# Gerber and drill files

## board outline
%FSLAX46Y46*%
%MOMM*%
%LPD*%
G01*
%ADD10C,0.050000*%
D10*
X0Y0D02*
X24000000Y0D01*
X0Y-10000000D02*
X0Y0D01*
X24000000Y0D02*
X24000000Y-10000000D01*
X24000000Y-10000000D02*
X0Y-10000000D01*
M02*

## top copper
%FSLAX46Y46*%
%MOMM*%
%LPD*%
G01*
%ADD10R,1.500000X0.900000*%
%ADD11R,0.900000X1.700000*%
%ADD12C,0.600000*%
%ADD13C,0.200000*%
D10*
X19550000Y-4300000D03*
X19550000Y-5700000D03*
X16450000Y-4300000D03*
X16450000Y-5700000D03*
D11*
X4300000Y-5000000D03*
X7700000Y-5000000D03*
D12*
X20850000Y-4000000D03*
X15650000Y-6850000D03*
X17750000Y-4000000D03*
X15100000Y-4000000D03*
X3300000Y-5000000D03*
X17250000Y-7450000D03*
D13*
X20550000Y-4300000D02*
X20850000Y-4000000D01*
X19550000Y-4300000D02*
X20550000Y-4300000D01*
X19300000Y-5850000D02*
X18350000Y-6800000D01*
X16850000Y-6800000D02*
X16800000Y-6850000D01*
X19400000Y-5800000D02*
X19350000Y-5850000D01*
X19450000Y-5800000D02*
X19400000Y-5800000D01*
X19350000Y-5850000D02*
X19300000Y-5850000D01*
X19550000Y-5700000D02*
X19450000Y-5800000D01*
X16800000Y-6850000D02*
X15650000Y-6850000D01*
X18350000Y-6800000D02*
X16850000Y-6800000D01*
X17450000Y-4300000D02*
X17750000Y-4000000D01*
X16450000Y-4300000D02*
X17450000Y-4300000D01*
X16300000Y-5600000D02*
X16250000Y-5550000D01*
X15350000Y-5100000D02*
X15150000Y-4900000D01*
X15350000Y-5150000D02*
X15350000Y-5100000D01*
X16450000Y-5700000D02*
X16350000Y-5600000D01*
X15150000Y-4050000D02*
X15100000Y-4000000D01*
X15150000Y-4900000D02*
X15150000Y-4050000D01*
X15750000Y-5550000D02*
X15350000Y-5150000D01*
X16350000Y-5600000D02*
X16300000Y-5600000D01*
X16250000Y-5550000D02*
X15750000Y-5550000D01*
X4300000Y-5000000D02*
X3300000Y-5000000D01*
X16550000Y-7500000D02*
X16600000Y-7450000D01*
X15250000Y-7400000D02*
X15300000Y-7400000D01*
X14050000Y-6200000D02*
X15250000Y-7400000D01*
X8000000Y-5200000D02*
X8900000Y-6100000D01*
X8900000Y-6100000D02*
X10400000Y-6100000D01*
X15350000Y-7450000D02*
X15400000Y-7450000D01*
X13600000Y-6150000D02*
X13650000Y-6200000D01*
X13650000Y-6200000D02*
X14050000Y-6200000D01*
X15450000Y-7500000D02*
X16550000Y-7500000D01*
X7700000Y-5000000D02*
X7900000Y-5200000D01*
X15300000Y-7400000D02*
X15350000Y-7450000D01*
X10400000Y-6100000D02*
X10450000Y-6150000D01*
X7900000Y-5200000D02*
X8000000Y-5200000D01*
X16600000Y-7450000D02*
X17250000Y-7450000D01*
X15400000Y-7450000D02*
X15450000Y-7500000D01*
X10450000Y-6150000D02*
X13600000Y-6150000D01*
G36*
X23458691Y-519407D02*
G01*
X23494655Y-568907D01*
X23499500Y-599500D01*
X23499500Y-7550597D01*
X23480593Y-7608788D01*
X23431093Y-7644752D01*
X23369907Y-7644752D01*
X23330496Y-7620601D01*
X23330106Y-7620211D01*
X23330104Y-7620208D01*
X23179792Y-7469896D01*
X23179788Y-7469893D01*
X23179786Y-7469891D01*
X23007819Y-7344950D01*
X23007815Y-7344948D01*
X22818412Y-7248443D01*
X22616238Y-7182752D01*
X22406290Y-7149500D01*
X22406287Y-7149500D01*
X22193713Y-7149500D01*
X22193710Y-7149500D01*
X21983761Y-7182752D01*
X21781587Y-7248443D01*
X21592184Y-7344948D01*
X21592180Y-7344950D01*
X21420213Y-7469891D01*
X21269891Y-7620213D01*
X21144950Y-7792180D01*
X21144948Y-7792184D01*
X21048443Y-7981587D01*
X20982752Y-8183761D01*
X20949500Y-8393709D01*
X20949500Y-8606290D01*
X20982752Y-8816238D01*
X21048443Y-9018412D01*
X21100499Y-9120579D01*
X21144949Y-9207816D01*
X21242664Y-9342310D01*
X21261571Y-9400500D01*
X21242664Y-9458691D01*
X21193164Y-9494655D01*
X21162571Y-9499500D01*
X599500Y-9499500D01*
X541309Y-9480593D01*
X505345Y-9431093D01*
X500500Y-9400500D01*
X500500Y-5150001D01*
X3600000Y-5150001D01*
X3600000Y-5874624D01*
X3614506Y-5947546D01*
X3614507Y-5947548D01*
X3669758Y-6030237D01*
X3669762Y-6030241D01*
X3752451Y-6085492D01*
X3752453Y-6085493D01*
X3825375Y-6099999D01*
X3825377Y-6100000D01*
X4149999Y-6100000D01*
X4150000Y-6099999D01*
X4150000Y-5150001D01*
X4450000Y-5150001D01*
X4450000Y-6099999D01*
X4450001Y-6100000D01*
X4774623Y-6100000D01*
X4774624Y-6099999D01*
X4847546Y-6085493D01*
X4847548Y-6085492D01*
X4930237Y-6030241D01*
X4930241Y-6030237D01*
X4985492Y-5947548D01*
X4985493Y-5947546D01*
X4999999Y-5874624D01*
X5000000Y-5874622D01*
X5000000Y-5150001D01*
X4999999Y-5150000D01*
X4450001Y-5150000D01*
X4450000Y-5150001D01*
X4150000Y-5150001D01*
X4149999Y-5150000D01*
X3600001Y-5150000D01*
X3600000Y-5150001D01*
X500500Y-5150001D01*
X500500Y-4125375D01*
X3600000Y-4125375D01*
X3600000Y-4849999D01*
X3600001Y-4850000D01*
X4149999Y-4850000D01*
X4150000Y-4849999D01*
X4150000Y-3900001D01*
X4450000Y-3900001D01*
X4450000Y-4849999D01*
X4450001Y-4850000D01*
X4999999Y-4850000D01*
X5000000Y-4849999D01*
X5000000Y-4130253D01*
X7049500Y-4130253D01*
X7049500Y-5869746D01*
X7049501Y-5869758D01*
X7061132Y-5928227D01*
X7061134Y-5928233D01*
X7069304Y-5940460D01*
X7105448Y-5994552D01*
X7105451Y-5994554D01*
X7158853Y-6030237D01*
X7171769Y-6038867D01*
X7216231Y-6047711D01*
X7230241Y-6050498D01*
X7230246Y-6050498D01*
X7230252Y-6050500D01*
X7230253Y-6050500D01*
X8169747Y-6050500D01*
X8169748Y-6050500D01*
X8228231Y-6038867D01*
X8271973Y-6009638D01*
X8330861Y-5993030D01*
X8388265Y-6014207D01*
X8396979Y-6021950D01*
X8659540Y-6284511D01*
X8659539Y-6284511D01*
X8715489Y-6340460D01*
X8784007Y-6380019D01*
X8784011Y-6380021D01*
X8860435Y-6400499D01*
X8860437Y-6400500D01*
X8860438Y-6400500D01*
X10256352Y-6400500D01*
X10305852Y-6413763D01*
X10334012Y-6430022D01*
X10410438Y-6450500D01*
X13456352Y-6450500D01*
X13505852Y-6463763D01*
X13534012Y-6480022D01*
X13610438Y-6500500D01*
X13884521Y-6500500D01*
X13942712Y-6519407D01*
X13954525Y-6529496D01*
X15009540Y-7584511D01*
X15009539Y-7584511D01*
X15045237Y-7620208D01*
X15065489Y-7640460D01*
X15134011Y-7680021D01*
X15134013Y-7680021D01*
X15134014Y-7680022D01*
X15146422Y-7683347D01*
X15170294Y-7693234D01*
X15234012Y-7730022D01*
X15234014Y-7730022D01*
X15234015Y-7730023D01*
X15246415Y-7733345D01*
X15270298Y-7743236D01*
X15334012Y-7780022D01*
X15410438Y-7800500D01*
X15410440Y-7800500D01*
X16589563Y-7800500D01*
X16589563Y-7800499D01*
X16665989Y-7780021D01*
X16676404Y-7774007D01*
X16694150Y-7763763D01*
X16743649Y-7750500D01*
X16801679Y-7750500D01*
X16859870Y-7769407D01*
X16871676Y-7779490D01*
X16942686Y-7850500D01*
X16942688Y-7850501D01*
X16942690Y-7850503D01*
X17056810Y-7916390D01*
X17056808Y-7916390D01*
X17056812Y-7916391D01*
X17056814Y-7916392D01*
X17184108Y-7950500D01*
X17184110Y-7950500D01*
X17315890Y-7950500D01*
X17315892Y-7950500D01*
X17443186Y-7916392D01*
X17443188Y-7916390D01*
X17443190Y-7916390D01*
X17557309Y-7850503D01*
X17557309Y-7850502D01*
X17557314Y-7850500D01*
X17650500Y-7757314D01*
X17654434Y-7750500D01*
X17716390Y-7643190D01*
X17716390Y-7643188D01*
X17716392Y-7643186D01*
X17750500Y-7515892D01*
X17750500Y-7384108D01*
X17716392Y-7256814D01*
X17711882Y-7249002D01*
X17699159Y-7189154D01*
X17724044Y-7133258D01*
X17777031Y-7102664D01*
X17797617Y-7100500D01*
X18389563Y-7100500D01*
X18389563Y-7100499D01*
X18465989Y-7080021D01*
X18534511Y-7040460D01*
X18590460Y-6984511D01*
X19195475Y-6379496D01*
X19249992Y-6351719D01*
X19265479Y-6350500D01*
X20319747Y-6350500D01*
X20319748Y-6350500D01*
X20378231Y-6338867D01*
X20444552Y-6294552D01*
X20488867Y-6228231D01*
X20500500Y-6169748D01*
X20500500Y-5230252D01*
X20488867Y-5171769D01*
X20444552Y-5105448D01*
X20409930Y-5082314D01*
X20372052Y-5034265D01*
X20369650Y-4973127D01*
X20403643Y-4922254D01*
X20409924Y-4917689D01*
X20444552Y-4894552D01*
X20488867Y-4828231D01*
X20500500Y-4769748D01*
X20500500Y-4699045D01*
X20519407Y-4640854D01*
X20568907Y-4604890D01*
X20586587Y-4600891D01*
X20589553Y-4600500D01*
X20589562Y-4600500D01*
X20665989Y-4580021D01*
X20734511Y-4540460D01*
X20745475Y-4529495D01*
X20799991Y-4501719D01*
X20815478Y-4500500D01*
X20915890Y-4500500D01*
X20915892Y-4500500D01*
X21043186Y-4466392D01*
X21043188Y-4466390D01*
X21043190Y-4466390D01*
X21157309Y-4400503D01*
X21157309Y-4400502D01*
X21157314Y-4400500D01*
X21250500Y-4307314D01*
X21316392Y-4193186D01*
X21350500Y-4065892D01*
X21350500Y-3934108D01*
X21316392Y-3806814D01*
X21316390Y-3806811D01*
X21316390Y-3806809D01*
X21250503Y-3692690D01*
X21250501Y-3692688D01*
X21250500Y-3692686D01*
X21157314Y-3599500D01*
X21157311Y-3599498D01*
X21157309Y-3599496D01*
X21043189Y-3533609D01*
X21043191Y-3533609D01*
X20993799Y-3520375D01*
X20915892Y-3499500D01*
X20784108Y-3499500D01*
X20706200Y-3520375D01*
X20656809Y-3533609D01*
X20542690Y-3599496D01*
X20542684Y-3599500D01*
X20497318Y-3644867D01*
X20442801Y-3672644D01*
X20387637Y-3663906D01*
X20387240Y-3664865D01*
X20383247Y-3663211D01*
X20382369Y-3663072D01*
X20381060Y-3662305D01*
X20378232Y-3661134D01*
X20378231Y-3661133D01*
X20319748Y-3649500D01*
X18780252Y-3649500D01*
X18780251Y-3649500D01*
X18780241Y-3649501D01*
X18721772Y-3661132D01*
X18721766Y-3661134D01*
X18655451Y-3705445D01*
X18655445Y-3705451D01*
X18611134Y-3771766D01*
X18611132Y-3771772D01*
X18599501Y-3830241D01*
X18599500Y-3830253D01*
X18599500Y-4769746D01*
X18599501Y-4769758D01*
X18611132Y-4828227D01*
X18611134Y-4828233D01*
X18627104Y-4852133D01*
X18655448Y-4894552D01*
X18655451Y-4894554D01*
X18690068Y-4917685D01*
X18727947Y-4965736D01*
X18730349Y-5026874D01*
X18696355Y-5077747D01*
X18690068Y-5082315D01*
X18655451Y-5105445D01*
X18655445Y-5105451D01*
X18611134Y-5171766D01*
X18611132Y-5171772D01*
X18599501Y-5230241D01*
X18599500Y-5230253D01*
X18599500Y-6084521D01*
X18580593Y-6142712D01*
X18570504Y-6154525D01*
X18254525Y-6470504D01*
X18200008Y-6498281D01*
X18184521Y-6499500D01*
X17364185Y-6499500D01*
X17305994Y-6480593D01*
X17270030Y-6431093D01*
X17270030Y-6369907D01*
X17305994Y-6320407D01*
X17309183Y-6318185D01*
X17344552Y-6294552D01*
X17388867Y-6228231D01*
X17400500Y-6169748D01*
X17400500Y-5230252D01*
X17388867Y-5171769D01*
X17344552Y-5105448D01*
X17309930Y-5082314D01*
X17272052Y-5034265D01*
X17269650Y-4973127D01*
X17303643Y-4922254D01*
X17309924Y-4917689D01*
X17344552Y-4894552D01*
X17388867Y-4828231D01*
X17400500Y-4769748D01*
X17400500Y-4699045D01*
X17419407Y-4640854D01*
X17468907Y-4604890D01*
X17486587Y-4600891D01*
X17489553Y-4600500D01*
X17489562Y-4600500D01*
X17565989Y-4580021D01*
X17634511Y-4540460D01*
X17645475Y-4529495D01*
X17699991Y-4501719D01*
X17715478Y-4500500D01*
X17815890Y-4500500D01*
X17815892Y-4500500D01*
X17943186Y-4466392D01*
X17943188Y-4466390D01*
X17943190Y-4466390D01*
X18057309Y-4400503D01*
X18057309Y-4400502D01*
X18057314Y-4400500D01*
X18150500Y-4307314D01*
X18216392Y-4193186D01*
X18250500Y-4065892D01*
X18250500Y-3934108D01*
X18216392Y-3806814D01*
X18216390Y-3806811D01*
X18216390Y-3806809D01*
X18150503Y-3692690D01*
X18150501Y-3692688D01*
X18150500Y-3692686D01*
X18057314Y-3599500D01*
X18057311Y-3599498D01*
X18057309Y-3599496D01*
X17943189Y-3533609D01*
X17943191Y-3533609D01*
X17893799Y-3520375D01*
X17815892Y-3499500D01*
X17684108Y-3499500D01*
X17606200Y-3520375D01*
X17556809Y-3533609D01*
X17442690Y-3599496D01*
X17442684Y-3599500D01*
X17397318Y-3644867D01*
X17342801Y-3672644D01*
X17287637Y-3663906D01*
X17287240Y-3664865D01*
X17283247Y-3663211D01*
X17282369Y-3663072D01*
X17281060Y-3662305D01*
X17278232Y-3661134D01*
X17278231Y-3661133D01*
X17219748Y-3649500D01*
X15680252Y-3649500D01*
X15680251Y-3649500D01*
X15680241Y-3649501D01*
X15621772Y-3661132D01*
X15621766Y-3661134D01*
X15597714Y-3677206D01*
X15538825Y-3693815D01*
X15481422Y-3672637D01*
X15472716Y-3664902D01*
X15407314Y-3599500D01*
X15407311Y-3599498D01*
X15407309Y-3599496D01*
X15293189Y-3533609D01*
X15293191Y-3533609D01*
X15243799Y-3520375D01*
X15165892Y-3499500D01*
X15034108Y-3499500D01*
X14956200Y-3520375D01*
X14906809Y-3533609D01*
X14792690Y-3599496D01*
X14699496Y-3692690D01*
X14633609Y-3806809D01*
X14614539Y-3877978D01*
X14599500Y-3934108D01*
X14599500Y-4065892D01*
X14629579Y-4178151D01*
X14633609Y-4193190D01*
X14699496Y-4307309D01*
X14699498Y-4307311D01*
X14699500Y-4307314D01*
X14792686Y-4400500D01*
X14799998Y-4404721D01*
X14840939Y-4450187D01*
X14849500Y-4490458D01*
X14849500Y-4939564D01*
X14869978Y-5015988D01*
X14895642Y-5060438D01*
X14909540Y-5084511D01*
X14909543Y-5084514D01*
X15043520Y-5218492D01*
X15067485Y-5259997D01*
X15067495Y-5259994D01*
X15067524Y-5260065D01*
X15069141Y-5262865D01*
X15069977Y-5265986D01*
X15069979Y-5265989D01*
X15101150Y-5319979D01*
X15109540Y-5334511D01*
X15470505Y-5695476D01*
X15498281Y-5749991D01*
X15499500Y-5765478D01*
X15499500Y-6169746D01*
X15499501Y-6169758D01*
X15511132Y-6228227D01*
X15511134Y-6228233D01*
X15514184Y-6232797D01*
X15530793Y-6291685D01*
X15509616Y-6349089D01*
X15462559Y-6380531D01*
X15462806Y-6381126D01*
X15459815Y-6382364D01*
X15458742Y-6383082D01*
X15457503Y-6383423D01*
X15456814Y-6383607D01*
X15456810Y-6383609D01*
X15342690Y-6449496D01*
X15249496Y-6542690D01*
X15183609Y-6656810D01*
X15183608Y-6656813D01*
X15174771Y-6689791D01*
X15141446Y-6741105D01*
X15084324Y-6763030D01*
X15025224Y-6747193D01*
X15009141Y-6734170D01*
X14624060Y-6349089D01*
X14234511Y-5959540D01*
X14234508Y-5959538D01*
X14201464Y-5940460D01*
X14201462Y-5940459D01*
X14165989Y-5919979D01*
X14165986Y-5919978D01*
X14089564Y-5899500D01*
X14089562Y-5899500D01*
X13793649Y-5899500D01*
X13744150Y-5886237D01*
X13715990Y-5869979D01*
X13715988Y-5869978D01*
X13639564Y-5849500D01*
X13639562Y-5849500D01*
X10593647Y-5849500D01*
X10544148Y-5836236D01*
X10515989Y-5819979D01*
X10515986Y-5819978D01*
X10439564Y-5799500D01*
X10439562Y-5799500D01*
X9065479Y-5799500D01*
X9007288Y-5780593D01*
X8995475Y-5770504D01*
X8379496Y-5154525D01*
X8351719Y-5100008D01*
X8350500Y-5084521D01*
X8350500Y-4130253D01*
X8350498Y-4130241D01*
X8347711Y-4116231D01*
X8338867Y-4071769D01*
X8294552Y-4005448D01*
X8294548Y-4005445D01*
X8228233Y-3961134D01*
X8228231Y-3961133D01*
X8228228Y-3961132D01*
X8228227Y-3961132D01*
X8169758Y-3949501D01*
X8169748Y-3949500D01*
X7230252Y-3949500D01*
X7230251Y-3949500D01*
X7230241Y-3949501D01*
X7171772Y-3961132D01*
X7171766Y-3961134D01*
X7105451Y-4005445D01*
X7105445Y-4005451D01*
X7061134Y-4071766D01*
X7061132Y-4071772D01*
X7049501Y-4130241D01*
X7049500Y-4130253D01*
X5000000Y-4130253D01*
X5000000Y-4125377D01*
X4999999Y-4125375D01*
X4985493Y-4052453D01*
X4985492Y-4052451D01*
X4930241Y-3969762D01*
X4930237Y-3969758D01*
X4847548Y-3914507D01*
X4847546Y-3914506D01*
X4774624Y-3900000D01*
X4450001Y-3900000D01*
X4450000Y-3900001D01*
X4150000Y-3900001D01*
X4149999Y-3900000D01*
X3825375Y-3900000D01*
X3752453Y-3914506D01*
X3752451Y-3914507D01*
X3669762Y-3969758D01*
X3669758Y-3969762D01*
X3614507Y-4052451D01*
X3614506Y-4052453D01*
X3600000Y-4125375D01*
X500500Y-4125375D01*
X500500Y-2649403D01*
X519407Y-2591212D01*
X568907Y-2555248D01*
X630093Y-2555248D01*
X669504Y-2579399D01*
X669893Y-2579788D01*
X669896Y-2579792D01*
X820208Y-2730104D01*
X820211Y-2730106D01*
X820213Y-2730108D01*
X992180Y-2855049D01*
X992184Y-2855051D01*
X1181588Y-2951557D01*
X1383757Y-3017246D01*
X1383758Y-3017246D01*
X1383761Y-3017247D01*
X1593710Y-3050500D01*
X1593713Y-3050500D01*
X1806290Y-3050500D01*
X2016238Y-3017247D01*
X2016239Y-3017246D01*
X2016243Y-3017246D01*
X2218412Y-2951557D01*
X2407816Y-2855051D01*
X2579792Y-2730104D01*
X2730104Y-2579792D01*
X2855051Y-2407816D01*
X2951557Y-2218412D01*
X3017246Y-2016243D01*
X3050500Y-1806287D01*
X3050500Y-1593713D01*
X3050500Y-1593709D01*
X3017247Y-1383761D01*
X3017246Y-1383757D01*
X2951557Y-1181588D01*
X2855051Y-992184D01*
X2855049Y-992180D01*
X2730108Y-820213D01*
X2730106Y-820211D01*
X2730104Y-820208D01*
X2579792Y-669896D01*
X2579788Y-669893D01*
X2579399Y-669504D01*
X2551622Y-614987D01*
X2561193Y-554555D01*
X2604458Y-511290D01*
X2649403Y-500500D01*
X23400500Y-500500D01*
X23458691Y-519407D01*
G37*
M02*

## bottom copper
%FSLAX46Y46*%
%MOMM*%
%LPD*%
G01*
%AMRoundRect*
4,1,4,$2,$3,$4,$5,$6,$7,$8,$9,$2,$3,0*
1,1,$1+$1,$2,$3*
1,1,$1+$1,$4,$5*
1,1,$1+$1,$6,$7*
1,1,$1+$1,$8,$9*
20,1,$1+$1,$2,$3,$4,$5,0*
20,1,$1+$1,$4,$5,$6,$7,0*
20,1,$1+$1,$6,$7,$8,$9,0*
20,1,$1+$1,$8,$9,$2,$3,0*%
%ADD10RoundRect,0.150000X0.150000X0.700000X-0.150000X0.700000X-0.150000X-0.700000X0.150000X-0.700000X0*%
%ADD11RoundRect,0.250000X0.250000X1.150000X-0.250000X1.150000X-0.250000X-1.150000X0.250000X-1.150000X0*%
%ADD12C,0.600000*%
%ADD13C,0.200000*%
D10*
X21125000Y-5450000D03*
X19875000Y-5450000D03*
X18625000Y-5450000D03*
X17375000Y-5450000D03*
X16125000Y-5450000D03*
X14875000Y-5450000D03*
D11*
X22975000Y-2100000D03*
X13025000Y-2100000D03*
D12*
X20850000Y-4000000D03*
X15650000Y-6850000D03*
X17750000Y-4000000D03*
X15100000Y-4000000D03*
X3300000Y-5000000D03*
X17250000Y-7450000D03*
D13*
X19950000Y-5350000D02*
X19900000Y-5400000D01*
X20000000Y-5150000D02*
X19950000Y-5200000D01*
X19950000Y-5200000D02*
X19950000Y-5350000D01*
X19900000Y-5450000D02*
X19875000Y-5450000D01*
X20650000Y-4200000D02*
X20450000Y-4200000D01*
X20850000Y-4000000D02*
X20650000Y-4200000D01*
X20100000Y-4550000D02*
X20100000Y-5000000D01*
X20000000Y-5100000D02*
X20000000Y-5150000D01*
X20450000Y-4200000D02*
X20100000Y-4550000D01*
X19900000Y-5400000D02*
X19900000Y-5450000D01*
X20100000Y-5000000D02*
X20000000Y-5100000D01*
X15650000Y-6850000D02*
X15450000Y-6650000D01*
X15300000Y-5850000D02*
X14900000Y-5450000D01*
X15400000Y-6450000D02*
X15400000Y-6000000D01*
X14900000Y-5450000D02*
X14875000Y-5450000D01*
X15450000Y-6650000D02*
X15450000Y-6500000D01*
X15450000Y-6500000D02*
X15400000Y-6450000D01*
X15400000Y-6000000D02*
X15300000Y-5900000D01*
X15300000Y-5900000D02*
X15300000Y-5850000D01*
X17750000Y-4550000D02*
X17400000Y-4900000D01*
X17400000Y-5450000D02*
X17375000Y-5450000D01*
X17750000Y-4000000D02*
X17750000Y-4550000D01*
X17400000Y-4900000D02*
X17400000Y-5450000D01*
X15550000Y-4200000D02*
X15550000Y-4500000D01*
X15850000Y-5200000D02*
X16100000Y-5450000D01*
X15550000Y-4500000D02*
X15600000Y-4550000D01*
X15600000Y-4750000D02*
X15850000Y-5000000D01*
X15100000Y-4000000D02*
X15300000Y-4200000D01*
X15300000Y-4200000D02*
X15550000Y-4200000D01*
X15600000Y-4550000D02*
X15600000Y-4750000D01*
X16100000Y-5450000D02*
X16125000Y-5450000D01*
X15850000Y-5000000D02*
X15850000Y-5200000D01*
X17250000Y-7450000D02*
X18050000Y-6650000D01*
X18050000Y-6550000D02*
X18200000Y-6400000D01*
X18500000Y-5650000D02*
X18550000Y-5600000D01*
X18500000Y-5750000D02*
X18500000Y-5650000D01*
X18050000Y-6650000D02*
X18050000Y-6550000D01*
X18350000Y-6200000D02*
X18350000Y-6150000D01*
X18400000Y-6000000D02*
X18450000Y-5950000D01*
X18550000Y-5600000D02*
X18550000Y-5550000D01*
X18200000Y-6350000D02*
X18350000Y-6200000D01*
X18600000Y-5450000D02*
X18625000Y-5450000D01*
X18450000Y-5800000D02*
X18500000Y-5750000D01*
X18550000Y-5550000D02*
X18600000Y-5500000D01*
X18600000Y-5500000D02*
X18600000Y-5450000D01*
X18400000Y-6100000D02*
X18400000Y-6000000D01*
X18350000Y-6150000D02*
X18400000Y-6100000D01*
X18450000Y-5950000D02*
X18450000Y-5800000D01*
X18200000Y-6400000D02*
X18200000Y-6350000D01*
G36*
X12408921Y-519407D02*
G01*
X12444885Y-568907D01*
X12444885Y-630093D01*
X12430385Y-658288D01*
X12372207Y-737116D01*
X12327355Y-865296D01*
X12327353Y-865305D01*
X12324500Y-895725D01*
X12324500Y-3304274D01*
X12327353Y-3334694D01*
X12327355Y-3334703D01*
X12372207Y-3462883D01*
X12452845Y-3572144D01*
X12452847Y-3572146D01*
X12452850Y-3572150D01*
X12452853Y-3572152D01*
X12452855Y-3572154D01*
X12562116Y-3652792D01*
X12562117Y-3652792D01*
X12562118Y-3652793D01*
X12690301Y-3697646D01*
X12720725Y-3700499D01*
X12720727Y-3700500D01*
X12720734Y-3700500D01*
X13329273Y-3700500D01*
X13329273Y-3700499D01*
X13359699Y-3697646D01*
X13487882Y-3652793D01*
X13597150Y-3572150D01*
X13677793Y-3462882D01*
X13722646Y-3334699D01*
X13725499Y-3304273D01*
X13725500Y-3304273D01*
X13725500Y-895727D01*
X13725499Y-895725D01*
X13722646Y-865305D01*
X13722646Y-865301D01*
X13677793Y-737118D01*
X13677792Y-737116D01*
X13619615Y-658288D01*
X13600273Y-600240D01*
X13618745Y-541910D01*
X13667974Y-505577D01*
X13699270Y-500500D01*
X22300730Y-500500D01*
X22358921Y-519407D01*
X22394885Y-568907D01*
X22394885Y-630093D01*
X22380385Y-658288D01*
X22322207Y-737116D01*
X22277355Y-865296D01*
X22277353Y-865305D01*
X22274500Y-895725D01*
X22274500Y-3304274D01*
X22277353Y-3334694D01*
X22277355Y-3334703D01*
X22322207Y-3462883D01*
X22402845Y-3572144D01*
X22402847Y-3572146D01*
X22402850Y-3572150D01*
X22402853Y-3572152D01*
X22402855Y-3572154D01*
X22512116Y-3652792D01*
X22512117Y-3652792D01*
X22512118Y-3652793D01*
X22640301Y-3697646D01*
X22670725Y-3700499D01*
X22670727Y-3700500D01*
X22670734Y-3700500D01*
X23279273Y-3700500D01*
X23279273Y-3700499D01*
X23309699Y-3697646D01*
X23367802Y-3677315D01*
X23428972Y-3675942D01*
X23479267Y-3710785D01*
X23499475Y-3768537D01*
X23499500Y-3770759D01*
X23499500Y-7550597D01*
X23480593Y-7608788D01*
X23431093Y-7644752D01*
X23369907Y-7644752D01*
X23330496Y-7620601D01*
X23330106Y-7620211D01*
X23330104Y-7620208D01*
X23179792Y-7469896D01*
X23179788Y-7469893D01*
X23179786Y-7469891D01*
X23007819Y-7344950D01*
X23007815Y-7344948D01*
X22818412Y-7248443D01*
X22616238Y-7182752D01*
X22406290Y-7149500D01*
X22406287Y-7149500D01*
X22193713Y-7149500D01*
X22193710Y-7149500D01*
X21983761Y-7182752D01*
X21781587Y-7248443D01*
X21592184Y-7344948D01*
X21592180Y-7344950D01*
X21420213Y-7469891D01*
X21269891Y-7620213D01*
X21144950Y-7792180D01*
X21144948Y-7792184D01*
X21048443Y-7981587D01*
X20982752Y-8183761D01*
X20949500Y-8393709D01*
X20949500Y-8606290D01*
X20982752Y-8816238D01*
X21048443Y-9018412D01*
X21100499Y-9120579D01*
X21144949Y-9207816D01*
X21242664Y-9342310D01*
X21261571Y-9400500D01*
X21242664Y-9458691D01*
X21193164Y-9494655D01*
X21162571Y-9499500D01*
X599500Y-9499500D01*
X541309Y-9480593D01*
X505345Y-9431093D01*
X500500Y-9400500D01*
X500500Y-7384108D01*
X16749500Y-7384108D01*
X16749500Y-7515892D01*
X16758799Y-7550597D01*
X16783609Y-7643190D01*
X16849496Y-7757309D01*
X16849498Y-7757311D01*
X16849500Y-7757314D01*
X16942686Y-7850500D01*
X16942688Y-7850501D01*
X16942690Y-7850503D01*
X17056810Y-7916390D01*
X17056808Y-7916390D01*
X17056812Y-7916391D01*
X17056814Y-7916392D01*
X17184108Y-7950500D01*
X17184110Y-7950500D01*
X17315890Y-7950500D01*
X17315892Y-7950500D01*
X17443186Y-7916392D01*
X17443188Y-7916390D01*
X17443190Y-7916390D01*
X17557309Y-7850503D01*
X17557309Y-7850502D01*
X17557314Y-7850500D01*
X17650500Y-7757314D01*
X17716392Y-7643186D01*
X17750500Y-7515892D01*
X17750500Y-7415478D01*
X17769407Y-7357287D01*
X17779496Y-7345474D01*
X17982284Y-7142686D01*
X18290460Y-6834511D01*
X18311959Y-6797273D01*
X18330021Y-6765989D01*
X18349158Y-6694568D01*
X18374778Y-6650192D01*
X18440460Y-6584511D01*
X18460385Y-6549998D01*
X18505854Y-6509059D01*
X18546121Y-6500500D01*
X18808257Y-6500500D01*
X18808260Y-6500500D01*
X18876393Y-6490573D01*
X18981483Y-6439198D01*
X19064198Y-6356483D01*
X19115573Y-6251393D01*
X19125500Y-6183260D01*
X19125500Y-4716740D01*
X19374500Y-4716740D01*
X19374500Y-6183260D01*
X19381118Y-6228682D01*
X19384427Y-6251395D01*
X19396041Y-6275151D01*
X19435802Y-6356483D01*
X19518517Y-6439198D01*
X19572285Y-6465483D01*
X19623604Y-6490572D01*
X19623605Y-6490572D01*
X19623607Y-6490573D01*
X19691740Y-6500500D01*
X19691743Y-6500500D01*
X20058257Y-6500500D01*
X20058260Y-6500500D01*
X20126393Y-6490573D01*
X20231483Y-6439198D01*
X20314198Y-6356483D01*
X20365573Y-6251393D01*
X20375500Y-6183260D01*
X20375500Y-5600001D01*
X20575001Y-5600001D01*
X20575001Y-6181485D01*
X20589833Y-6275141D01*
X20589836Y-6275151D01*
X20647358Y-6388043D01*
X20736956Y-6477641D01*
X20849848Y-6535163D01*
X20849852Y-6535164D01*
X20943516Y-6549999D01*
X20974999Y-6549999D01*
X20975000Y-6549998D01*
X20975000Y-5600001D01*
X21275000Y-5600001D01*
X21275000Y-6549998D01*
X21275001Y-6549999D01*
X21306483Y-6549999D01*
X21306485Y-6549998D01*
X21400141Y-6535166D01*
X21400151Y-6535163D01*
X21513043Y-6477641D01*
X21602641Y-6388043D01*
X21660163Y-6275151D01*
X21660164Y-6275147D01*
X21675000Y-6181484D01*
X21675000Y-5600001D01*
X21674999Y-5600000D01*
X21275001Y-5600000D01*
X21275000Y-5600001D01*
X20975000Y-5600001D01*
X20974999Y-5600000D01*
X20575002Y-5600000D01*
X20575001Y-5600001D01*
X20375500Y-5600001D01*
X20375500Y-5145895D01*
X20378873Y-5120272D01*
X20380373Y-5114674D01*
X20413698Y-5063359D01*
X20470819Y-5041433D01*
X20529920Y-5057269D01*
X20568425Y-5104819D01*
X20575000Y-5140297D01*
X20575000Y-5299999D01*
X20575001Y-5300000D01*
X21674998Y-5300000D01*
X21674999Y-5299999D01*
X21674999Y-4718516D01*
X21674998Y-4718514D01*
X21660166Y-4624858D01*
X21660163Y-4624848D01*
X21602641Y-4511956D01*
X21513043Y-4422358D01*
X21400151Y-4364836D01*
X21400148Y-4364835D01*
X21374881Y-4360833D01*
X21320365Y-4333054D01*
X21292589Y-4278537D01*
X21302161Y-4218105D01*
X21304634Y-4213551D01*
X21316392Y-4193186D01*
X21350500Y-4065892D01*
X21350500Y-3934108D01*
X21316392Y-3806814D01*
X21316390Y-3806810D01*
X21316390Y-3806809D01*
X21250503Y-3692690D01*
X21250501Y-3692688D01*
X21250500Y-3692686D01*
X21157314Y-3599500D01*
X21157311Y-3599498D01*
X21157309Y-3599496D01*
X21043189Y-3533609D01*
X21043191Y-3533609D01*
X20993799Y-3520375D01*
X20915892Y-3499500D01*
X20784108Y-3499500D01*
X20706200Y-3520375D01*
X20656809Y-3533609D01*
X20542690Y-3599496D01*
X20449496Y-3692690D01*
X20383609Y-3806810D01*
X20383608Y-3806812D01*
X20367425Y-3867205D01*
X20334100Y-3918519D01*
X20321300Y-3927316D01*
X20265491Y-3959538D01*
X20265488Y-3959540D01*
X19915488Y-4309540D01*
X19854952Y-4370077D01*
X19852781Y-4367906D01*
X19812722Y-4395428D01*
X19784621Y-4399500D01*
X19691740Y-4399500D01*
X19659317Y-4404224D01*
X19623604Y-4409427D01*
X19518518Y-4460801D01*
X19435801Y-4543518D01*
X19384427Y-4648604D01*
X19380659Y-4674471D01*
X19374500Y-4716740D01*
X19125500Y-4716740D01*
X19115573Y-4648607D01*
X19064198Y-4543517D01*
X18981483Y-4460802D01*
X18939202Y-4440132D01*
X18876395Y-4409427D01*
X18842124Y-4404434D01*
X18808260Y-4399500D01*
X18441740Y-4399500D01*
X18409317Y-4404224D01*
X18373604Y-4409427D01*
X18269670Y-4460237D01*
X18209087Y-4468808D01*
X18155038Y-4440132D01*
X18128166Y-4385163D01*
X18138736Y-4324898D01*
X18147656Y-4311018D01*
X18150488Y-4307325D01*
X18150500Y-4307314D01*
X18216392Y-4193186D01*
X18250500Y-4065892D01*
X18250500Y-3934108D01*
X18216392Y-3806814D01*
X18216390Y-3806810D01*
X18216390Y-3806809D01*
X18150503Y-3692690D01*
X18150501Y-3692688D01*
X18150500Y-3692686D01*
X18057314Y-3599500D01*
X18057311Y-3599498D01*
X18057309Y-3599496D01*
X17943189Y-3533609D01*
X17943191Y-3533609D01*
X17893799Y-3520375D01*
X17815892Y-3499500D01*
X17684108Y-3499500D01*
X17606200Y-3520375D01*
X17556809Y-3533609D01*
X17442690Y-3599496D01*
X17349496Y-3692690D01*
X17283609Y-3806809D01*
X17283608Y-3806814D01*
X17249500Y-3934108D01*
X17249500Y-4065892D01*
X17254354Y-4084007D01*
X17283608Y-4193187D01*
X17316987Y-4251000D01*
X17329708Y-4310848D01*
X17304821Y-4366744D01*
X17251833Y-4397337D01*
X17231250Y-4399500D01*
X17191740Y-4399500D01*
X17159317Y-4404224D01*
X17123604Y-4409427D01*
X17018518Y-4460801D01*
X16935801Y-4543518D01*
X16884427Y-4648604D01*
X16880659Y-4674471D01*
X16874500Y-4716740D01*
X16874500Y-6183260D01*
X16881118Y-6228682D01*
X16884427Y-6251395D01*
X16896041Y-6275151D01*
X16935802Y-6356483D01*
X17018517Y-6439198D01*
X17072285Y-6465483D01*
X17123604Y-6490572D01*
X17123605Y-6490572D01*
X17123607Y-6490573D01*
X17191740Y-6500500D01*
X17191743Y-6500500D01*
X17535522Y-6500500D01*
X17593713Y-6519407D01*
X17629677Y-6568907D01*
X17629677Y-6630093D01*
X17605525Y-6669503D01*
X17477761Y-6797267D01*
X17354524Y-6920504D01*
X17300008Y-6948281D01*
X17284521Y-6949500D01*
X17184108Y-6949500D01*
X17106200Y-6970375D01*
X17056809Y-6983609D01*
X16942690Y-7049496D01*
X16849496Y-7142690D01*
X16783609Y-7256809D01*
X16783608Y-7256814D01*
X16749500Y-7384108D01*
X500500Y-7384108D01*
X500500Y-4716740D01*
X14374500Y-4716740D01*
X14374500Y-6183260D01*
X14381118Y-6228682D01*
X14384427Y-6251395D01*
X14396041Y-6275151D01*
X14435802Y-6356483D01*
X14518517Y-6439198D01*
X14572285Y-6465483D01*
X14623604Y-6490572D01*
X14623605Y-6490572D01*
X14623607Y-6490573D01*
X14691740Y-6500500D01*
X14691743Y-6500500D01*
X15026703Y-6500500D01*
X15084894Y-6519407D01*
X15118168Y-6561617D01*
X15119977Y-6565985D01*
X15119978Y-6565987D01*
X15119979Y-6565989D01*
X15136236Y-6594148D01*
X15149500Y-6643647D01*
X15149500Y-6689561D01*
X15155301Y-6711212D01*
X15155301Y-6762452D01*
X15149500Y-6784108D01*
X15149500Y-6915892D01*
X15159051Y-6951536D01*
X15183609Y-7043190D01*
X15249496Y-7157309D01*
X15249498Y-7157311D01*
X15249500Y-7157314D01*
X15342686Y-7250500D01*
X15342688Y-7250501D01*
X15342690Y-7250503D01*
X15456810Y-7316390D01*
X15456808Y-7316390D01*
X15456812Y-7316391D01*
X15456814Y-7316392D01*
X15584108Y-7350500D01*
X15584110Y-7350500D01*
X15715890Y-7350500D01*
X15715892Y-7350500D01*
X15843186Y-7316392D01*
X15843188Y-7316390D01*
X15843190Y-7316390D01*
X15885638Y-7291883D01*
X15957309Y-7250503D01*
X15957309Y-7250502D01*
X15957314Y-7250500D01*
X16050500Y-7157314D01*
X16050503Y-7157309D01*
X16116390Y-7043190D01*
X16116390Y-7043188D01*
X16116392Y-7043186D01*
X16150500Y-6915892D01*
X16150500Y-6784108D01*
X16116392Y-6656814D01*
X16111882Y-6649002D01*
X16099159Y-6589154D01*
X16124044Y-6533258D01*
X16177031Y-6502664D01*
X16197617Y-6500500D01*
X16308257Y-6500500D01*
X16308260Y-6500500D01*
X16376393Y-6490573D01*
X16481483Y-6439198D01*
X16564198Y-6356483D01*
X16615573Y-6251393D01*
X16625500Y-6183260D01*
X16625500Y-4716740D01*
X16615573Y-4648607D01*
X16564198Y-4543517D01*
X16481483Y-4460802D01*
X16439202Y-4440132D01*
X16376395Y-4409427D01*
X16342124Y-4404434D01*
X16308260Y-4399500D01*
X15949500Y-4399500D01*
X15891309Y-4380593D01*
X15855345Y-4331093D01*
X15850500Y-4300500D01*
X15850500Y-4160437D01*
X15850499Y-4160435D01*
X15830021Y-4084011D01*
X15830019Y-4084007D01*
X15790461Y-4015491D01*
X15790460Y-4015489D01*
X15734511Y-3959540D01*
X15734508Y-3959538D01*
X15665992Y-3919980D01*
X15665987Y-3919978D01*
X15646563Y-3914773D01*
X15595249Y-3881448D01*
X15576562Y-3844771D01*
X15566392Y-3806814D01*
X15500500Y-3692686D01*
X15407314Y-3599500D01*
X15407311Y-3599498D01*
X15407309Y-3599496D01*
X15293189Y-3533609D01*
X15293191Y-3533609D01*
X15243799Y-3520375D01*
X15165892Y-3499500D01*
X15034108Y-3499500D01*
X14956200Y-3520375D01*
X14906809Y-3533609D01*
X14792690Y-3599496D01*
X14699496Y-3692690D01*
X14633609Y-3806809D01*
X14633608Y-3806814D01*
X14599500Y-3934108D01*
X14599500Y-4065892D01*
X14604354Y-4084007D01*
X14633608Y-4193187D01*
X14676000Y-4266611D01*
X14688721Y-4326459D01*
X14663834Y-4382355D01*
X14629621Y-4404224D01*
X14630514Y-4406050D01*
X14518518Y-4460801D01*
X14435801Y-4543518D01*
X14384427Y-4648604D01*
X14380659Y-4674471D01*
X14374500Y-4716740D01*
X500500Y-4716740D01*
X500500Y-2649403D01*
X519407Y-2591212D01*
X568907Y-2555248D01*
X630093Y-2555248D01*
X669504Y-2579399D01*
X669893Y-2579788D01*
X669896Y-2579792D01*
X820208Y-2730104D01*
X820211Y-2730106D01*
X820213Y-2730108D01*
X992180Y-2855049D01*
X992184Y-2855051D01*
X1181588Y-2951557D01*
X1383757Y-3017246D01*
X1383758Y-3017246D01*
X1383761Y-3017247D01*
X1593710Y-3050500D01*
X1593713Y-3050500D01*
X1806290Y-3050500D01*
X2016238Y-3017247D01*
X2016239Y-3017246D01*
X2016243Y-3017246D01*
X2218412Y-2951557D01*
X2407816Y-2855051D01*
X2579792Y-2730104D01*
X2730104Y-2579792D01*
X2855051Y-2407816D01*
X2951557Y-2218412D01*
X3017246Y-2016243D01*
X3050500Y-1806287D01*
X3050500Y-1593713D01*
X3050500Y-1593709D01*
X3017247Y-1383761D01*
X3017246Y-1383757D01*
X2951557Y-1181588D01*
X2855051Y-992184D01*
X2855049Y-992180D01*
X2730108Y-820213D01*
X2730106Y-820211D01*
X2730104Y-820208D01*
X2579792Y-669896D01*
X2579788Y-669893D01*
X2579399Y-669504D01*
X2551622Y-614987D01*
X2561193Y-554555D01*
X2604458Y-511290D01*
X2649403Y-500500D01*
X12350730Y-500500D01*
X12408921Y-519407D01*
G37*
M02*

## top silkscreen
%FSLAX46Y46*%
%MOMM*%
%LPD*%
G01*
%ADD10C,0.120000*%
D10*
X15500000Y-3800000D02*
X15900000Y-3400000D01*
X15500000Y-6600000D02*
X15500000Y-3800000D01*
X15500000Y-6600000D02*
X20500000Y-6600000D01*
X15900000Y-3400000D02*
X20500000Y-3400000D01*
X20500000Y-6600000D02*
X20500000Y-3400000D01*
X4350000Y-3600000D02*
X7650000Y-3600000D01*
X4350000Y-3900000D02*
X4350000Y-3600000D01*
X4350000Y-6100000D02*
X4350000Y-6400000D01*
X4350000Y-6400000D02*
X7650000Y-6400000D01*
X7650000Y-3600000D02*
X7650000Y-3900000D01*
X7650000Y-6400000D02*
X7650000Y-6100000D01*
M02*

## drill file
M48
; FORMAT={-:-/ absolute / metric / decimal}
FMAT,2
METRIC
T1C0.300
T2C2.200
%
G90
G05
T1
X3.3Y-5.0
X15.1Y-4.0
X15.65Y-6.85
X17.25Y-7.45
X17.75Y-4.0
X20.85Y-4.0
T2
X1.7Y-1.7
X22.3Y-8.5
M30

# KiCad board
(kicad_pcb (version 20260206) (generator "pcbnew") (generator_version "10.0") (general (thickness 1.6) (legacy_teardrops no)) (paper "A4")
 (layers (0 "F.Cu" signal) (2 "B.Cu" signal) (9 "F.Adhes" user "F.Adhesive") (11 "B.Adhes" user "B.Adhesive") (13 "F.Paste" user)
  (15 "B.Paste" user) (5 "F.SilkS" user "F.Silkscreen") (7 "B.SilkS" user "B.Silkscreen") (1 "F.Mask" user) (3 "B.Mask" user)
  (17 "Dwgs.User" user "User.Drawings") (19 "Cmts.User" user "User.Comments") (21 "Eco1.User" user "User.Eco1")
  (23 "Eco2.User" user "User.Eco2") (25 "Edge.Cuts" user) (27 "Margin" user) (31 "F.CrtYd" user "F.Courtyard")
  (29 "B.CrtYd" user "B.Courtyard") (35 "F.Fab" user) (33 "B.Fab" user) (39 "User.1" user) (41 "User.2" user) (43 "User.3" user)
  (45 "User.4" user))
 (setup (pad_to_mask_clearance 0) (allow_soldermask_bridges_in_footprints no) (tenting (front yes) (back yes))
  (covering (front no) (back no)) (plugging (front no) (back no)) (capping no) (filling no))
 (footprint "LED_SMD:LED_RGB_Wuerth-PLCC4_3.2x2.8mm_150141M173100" (layer "F.Cu") (at 18 5)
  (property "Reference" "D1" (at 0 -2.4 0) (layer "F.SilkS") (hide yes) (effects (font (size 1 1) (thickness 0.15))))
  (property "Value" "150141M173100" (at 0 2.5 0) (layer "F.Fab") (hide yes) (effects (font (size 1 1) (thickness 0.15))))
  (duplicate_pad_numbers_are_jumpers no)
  (fp_line (start -2.5 -1.2) (end -2.1 -1.6) (stroke (width 0.12) (type default)) (layer "F.SilkS"))
  (fp_line (start -2.5 1.6) (end -2.5 -1.2) (stroke (width 0.12) (type solid)) (layer "F.SilkS"))
  (fp_line (start -2.5 1.6) (end 2.5 1.6) (stroke (width 0.12) (type solid)) (layer "F.SilkS"))
  (fp_line (start -2.1 -1.6) (end 2.5 -1.6) (stroke (width 0.12) (type solid)) (layer "F.SilkS"))
  (fp_line (start 2.5 1.6) (end 2.5 -1.6) (stroke (width 0.12) (type solid)) (layer "F.SilkS"))
  (pad "1" smd rect (at 1.55 -0.7) (size 1.5 0.9) (layers "F.Cu" "F.Mask" "F.Paste") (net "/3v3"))
  (pad "2" smd rect (at 1.55 0.7) (size 1.5 0.9) (layers "F.Cu" "F.Mask" "F.Paste") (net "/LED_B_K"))
  (pad "3" smd rect (at -1.55 -0.7) (size 1.5 0.9) (layers "F.Cu" "F.Mask" "F.Paste") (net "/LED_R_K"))
  (pad "4" smd rect (at -1.55 0.7) (size 1.5 0.9) (layers "F.Cu" "F.Mask" "F.Paste") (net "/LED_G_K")))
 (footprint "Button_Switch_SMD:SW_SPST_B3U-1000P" (layer "F.Cu") (at 6 5)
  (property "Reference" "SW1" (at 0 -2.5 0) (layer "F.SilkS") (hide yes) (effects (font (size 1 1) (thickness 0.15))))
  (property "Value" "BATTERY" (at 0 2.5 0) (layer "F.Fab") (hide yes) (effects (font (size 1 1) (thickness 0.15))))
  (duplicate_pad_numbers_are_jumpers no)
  (fp_line (start -1.65 -1.4) (end 1.65 -1.4) (stroke (width 0.12) (type solid)) (layer "F.SilkS"))
  (fp_line (start -1.65 -1.1) (end -1.65 -1.4) (stroke (width 0.12) (type solid)) (layer "F.SilkS"))
  (fp_line (start -1.65 1.1) (end -1.65 1.4) (stroke (width 0.12) (type solid)) (layer "F.SilkS"))
  (fp_line (start -1.65 1.4) (end 1.65 1.4) (stroke (width 0.12) (type solid)) (layer "F.SilkS"))
  (fp_line (start 1.65 -1.4) (end 1.65 -1.1) (stroke (width 0.12) (type solid)) (layer "F.SilkS"))
  (fp_line (start 1.65 1.4) (end 1.65 1.1) (stroke (width 0.12) (type solid)) (layer "F.SilkS"))
  (pad "1" smd rect (at -1.7 0) (size 0.9 1.7) (layers "F.Cu" "F.Mask" "F.Paste") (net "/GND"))
  (pad "2" smd rect (at 1.7 0) (size 0.9 1.7) (layers "F.Cu" "F.Mask" "F.Paste") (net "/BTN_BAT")))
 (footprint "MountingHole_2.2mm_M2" (layer "F.Cu") (at 22.3 8.5)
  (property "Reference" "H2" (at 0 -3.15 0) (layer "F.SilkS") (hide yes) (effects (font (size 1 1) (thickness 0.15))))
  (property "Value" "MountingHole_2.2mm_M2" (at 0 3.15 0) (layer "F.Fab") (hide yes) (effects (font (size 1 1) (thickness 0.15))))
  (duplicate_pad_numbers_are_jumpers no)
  (pad "" np_thru_hole circle (at 0 0) (size 2.2 2.2) (drill 2.2) (layers "*.Cu" "*.Mask")))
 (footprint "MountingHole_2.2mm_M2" (layer "F.Cu") (at 1.7 1.7)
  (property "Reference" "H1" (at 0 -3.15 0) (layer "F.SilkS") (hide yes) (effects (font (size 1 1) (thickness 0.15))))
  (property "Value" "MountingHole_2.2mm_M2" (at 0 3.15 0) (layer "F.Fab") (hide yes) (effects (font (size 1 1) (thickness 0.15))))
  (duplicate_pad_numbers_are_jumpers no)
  (pad "" np_thru_hole circle (at 0 0) (size 2.2 2.2) (drill 2.2) (layers "*.Cu" "*.Mask")))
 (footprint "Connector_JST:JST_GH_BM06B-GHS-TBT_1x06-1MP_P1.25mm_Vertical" (layer "B.Cu") (at 18 3.5 180)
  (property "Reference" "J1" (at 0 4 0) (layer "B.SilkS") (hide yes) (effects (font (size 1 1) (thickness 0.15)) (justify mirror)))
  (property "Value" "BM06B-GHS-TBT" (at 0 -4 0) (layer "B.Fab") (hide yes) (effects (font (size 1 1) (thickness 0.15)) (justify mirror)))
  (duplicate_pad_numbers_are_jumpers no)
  (pad "1" smd roundrect (at -3.125 -1.95 180) (size 0.6 1.7) (layers "B.Cu" "B.Mask" "B.Paste") (roundrect_rratio 0.25) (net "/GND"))
  (pad "2" smd roundrect (at -1.875 -1.95 180) (size 0.6 1.7) (layers "B.Cu" "B.Mask" "B.Paste") (roundrect_rratio 0.25) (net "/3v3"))
  (pad "3" smd roundrect (at -0.625 -1.95 180) (size 0.6 1.7) (layers "B.Cu" "B.Mask" "B.Paste") (roundrect_rratio 0.25) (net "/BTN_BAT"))
  (pad "4" smd roundrect (at 0.625 -1.95 180) (size 0.6 1.7) (layers "B.Cu" "B.Mask" "B.Paste") (roundrect_rratio 0.25) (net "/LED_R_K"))
  (pad "5" smd roundrect (at 1.875 -1.95 180) (size 0.6 1.7) (layers "B.Cu" "B.Mask" "B.Paste") (roundrect_rratio 0.25) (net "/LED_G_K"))
  (pad "6" smd roundrect (at 3.125 -1.95 180) (size 0.6 1.7) (layers "B.Cu" "B.Mask" "B.Paste") (roundrect_rratio 0.25) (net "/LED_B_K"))
  (pad "MP" smd roundrect (at -4.975 1.4 180) (size 1 2.8) (layers "B.Cu" "B.Mask" "B.Paste") (roundrect_rratio 0.25))
  (pad "MP" smd roundrect (at 4.975 1.4 180) (size 1 2.8) (layers "B.Cu" "B.Mask" "B.Paste") (roundrect_rratio 0.25)))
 (gr_line (start 0 0) (end 24 0) (stroke (width 0.05) (type default)) (layer "Edge.Cuts"))
 (gr_line (start 0 10) (end 0 0) (stroke (width 0.05) (type default)) (layer "Edge.Cuts"))
 (gr_line (start 24 0) (end 24 10) (stroke (width 0.05) (type default)) (layer "Edge.Cuts"))
 (gr_line (start 24 10) (end 0 10) (stroke (width 0.05) (type default)) (layer "Edge.Cuts"))
 (segment (start 20.55 4.3) (end 20.85 4) (width 0.2) (layer "F.Cu") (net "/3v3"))
 (segment (start 19.55 4.3) (end 20.55 4.3) (width 0.2) (layer "F.Cu") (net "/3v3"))
 (via (at 20.85 4) (size 0.6) (drill 0.3) (layers "F.Cu" "B.Cu") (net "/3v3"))
 (segment (start 19.95 5.35) (end 19.9 5.4) (width 0.2) (layer "B.Cu") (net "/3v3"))
 (segment (start 20 5.15) (end 19.95 5.2) (width 0.2) (layer "B.Cu") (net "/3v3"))
 (segment (start 19.95 5.2) (end 19.95 5.35) (width 0.2) (layer "B.Cu") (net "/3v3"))
 (segment (start 19.9 5.45) (end 19.875 5.45) (width 0.2) (layer "B.Cu") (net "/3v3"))
 (segment (start 20.65 4.2) (end 20.45 4.2) (width 0.2) (layer "B.Cu") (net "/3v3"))
 (segment (start 20.85 4) (end 20.65 4.2) (width 0.2) (layer "B.Cu") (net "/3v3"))
 (segment (start 20.1 4.55) (end 20.1 5) (width 0.2) (layer "B.Cu") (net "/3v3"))
 (segment (start 20 5.1) (end 20 5.15) (width 0.2) (layer "B.Cu") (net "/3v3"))
 (segment (start 20.45 4.2) (end 20.1 4.55) (width 0.2) (layer "B.Cu") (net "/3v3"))
 (segment (start 19.9 5.4) (end 19.9 5.45) (width 0.2) (layer "B.Cu") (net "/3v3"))
 (segment (start 20.1 5) (end 20 5.1) (width 0.2) (layer "B.Cu") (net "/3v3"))
 (segment (start 19.3 5.85) (end 18.35 6.8) (width 0.2) (layer "F.Cu") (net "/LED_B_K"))
 (segment (start 16.85 6.8) (end 16.8 6.85) (width 0.2) (layer "F.Cu") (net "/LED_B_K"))
 (segment (start 19.4 5.8) (end 19.35 5.85) (width 0.2) (layer "F.Cu") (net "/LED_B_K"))
 (segment (start 19.45 5.8) (end 19.4 5.8) (width 0.2) (layer "F.Cu") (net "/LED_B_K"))
 (segment (start 19.35 5.85) (end 19.3 5.85) (width 0.2) (layer "F.Cu") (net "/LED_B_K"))
 (segment (start 19.55 5.7) (end 19.45 5.8) (width 0.2) (layer "F.Cu") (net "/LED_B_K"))
 (segment (start 16.8 6.85) (end 15.65 6.85) (width 0.2) (layer "F.Cu") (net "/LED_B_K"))
 (segment (start 18.35 6.8) (end 16.85 6.8) (width 0.2) (layer "F.Cu") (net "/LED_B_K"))
 (via (at 15.65 6.85) (size 0.6) (drill 0.3) (layers "F.Cu" "B.Cu") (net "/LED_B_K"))
 (segment (start 15.65 6.85) (end 15.45 6.65) (width 0.2) (layer "B.Cu") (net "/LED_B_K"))
 (segment (start 15.3 5.85) (end 14.9 5.45) (width 0.2) (layer "B.Cu") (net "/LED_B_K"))
 (segment (start 15.4 6.45) (end 15.4 6) (width 0.2) (layer "B.Cu") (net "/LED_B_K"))
 (segment (start 14.9 5.45) (end 14.875 5.45) (width 0.2) (layer "B.Cu") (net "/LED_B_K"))
 (segment (start 15.45 6.65) (end 15.45 6.5) (width 0.2) (layer "B.Cu") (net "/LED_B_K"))
 (segment (start 15.45 6.5) (end 15.4 6.45) (width 0.2) (layer "B.Cu") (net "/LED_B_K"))
 (segment (start 15.4 6) (end 15.3 5.9) (width 0.2) (layer "B.Cu") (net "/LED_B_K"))
 (segment (start 15.3 5.9) (end 15.3 5.85) (width 0.2) (layer "B.Cu") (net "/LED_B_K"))
 (segment (start 17.45 4.3) (end 17.75 4) (width 0.2) (layer "F.Cu") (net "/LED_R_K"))
 (segment (start 16.45 4.3) (end 17.45 4.3) (width 0.2) (layer "F.Cu") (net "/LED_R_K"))
 (via (at 17.75 4) (size 0.6) (drill 0.3) (layers "F.Cu" "B.Cu") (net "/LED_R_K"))
 (segment (start 17.75 4.55) (end 17.4 4.9) (width 0.2) (layer "B.Cu") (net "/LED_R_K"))
 (segment (start 17.4 5.45) (end 17.375 5.45) (width 0.2) (layer "B.Cu") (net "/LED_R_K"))
 (segment (start 17.75 4) (end 17.75 4.55) (width 0.2) (layer "B.Cu") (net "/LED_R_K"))
 (segment (start 17.4 4.9) (end 17.4 5.45) (width 0.2) (layer "B.Cu") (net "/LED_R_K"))
 (segment (start 16.3 5.6) (end 16.25 5.55) (width 0.2) (layer "F.Cu") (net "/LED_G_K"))
 (segment (start 15.35 5.1) (end 15.15 4.9) (width 0.2) (layer "F.Cu") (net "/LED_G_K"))
 (segment (start 15.35 5.15) (end 15.35 5.1) (width 0.2) (layer "F.Cu") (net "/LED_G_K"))
 (segment (start 16.45 5.7) (end 16.35 5.6) (width 0.2) (layer "F.Cu") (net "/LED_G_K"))
 (segment (start 15.15 4.05) (end 15.1 4) (width 0.2) (layer "F.Cu") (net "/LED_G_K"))
 (segment (start 15.15 4.9) (end 15.15 4.05) (width 0.2) (layer "F.Cu") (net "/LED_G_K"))
 (segment (start 15.75 5.55) (end 15.35 5.15) (width 0.2) (layer "F.Cu") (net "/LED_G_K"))
 (segment (start 16.35 5.6) (end 16.3 5.6) (width 0.2) (layer "F.Cu") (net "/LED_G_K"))
 (segment (start 16.25 5.55) (end 15.75 5.55) (width 0.2) (layer "F.Cu") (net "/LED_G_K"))
 (via (at 15.1 4) (size 0.6) (drill 0.3) (layers "F.Cu" "B.Cu") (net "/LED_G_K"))
 (segment (start 15.55 4.2) (end 15.55 4.5) (width 0.2) (layer "B.Cu") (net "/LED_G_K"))
 (segment (start 15.85 5.2) (end 16.1 5.45) (width 0.2) (layer "B.Cu") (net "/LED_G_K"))
 (segment (start 15.55 4.5) (end 15.6 4.55) (width 0.2) (layer "B.Cu") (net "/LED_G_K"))
 (segment (start 15.6 4.75) (end 15.85 5) (width 0.2) (layer "B.Cu") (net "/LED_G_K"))
 (segment (start 15.1 4) (end 15.3 4.2) (width 0.2) (layer "B.Cu") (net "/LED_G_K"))
 (segment (start 15.3 4.2) (end 15.55 4.2) (width 0.2) (layer "B.Cu") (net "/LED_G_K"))
 (segment (start 15.6 4.55) (end 15.6 4.75) (width 0.2) (layer "B.Cu") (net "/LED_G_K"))
 (segment (start 16.1 5.45) (end 16.125 5.45) (width 0.2) (layer "B.Cu") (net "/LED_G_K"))
 (segment (start 15.85 5) (end 15.85 5.2) (width 0.2) (layer "B.Cu") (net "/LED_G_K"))
 (segment (start 4.3 5) (end 3.3 5) (width 0.2) (layer "F.Cu") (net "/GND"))
 (via (at 3.3 5) (size 0.6) (drill 0.3) (layers "F.Cu" "B.Cu") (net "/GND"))
 (segment (start 16.55 7.5) (end 16.6 7.45) (width 0.2) (layer "F.Cu") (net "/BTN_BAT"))
 (segment (start 15.25 7.4) (end 15.3 7.4) (width 0.2) (layer "F.Cu") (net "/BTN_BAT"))
 (segment (start 14.05 6.2) (end 15.25 7.4) (width 0.2) (layer "F.Cu") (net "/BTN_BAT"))
 (segment (start 8 5.2) (end 8.9 6.1) (width 0.2) (layer "F.Cu") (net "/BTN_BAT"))
 (segment (start 8.9 6.1) (end 10.4 6.1) (width 0.2) (layer "F.Cu") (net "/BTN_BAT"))
 (segment (start 15.35 7.45) (end 15.4 7.45) (width 0.2) (layer "F.Cu") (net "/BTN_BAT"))
 (segment (start 13.6 6.15) (end 13.65 6.2) (width 0.2) (layer "F.Cu") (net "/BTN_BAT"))
 (segment (start 13.65 6.2) (end 14.05 6.2) (width 0.2) (layer "F.Cu") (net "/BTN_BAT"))
 (segment (start 15.45 7.5) (end 16.55 7.5) (width 0.2) (layer "F.Cu") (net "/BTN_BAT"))
 (segment (start 7.7 5) (end 7.9 5.2) (width 0.2) (layer "F.Cu") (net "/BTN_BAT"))
 (segment (start 15.3 7.4) (end 15.35 7.45) (width 0.2) (layer "F.Cu") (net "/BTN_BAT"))
 (segment (start 10.4 6.1) (end 10.45 6.15) (width 0.2) (layer "F.Cu") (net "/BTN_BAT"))
 (segment (start 7.9 5.2) (end 8 5.2) (width 0.2) (layer "F.Cu") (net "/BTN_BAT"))
 (segment (start 16.6 7.45) (end 17.25 7.45) (width 0.2) (layer "F.Cu") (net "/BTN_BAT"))
 (segment (start 15.4 7.45) (end 15.45 7.5) (width 0.2) (layer "F.Cu") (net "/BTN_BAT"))
 (segment (start 10.45 6.15) (end 13.6 6.15) (width 0.2) (layer "F.Cu") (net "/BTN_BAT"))
 (via (at 17.25 7.45) (size 0.6) (drill 0.3) (layers "F.Cu" "B.Cu") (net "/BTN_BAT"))
 (segment (start 17.25 7.45) (end 18.05 6.65) (width 0.2) (layer "B.Cu") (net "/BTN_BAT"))
 (segment (start 18.05 6.55) (end 18.2 6.4) (width 0.2) (layer "B.Cu") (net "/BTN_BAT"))
 (segment (start 18.5 5.65) (end 18.55 5.6) (width 0.2) (layer "B.Cu") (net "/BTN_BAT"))
 (segment (start 18.5 5.75) (end 18.5 5.65) (width 0.2) (layer "B.Cu") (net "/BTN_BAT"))
 (segment (start 18.05 6.65) (end 18.05 6.55) (width 0.2) (layer "B.Cu") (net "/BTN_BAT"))
 (segment (start 18.35 6.2) (end 18.35 6.15) (width 0.2) (layer "B.Cu") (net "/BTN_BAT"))
 (segment (start 18.4 6) (end 18.45 5.95) (width 0.2) (layer "B.Cu") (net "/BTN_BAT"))
 (segment (start 18.55 5.6) (end 18.55 5.55) (width 0.2) (layer "B.Cu") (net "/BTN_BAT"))
 (segment (start 18.2 6.35) (end 18.35 6.2) (width 0.2) (layer "B.Cu") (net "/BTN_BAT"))
 (segment (start 18.6 5.45) (end 18.625 5.45) (width 0.2) (layer "B.Cu") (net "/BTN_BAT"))
 (segment (start 18.45 5.8) (end 18.5 5.75) (width 0.2) (layer "B.Cu") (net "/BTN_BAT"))
 (segment (start 18.55 5.55) (end 18.6 5.5) (width 0.2) (layer "B.Cu") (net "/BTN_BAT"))
 (segment (start 18.6 5.5) (end 18.6 5.45) (width 0.2) (layer "B.Cu") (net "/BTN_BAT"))
 (segment (start 18.4 6.1) (end 18.4 6) (width 0.2) (layer "B.Cu") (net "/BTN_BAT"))
 (segment (start 18.35 6.15) (end 18.4 6.1) (width 0.2) (layer "B.Cu") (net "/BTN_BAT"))
 (segment (start 18.45 5.95) (end 18.45 5.8) (width 0.2) (layer "B.Cu") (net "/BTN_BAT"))
 (segment (start 18.2 6.4) (end 18.2 6.35) (width 0.2) (layer "B.Cu") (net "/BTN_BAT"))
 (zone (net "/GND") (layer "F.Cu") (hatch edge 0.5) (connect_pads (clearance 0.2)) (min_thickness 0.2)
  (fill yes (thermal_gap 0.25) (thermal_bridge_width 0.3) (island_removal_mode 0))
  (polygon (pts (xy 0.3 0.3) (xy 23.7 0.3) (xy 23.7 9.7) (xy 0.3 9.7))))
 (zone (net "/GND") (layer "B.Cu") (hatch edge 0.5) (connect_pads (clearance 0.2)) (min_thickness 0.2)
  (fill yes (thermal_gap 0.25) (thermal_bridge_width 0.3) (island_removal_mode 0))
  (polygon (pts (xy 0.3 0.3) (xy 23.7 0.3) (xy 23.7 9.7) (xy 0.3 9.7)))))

